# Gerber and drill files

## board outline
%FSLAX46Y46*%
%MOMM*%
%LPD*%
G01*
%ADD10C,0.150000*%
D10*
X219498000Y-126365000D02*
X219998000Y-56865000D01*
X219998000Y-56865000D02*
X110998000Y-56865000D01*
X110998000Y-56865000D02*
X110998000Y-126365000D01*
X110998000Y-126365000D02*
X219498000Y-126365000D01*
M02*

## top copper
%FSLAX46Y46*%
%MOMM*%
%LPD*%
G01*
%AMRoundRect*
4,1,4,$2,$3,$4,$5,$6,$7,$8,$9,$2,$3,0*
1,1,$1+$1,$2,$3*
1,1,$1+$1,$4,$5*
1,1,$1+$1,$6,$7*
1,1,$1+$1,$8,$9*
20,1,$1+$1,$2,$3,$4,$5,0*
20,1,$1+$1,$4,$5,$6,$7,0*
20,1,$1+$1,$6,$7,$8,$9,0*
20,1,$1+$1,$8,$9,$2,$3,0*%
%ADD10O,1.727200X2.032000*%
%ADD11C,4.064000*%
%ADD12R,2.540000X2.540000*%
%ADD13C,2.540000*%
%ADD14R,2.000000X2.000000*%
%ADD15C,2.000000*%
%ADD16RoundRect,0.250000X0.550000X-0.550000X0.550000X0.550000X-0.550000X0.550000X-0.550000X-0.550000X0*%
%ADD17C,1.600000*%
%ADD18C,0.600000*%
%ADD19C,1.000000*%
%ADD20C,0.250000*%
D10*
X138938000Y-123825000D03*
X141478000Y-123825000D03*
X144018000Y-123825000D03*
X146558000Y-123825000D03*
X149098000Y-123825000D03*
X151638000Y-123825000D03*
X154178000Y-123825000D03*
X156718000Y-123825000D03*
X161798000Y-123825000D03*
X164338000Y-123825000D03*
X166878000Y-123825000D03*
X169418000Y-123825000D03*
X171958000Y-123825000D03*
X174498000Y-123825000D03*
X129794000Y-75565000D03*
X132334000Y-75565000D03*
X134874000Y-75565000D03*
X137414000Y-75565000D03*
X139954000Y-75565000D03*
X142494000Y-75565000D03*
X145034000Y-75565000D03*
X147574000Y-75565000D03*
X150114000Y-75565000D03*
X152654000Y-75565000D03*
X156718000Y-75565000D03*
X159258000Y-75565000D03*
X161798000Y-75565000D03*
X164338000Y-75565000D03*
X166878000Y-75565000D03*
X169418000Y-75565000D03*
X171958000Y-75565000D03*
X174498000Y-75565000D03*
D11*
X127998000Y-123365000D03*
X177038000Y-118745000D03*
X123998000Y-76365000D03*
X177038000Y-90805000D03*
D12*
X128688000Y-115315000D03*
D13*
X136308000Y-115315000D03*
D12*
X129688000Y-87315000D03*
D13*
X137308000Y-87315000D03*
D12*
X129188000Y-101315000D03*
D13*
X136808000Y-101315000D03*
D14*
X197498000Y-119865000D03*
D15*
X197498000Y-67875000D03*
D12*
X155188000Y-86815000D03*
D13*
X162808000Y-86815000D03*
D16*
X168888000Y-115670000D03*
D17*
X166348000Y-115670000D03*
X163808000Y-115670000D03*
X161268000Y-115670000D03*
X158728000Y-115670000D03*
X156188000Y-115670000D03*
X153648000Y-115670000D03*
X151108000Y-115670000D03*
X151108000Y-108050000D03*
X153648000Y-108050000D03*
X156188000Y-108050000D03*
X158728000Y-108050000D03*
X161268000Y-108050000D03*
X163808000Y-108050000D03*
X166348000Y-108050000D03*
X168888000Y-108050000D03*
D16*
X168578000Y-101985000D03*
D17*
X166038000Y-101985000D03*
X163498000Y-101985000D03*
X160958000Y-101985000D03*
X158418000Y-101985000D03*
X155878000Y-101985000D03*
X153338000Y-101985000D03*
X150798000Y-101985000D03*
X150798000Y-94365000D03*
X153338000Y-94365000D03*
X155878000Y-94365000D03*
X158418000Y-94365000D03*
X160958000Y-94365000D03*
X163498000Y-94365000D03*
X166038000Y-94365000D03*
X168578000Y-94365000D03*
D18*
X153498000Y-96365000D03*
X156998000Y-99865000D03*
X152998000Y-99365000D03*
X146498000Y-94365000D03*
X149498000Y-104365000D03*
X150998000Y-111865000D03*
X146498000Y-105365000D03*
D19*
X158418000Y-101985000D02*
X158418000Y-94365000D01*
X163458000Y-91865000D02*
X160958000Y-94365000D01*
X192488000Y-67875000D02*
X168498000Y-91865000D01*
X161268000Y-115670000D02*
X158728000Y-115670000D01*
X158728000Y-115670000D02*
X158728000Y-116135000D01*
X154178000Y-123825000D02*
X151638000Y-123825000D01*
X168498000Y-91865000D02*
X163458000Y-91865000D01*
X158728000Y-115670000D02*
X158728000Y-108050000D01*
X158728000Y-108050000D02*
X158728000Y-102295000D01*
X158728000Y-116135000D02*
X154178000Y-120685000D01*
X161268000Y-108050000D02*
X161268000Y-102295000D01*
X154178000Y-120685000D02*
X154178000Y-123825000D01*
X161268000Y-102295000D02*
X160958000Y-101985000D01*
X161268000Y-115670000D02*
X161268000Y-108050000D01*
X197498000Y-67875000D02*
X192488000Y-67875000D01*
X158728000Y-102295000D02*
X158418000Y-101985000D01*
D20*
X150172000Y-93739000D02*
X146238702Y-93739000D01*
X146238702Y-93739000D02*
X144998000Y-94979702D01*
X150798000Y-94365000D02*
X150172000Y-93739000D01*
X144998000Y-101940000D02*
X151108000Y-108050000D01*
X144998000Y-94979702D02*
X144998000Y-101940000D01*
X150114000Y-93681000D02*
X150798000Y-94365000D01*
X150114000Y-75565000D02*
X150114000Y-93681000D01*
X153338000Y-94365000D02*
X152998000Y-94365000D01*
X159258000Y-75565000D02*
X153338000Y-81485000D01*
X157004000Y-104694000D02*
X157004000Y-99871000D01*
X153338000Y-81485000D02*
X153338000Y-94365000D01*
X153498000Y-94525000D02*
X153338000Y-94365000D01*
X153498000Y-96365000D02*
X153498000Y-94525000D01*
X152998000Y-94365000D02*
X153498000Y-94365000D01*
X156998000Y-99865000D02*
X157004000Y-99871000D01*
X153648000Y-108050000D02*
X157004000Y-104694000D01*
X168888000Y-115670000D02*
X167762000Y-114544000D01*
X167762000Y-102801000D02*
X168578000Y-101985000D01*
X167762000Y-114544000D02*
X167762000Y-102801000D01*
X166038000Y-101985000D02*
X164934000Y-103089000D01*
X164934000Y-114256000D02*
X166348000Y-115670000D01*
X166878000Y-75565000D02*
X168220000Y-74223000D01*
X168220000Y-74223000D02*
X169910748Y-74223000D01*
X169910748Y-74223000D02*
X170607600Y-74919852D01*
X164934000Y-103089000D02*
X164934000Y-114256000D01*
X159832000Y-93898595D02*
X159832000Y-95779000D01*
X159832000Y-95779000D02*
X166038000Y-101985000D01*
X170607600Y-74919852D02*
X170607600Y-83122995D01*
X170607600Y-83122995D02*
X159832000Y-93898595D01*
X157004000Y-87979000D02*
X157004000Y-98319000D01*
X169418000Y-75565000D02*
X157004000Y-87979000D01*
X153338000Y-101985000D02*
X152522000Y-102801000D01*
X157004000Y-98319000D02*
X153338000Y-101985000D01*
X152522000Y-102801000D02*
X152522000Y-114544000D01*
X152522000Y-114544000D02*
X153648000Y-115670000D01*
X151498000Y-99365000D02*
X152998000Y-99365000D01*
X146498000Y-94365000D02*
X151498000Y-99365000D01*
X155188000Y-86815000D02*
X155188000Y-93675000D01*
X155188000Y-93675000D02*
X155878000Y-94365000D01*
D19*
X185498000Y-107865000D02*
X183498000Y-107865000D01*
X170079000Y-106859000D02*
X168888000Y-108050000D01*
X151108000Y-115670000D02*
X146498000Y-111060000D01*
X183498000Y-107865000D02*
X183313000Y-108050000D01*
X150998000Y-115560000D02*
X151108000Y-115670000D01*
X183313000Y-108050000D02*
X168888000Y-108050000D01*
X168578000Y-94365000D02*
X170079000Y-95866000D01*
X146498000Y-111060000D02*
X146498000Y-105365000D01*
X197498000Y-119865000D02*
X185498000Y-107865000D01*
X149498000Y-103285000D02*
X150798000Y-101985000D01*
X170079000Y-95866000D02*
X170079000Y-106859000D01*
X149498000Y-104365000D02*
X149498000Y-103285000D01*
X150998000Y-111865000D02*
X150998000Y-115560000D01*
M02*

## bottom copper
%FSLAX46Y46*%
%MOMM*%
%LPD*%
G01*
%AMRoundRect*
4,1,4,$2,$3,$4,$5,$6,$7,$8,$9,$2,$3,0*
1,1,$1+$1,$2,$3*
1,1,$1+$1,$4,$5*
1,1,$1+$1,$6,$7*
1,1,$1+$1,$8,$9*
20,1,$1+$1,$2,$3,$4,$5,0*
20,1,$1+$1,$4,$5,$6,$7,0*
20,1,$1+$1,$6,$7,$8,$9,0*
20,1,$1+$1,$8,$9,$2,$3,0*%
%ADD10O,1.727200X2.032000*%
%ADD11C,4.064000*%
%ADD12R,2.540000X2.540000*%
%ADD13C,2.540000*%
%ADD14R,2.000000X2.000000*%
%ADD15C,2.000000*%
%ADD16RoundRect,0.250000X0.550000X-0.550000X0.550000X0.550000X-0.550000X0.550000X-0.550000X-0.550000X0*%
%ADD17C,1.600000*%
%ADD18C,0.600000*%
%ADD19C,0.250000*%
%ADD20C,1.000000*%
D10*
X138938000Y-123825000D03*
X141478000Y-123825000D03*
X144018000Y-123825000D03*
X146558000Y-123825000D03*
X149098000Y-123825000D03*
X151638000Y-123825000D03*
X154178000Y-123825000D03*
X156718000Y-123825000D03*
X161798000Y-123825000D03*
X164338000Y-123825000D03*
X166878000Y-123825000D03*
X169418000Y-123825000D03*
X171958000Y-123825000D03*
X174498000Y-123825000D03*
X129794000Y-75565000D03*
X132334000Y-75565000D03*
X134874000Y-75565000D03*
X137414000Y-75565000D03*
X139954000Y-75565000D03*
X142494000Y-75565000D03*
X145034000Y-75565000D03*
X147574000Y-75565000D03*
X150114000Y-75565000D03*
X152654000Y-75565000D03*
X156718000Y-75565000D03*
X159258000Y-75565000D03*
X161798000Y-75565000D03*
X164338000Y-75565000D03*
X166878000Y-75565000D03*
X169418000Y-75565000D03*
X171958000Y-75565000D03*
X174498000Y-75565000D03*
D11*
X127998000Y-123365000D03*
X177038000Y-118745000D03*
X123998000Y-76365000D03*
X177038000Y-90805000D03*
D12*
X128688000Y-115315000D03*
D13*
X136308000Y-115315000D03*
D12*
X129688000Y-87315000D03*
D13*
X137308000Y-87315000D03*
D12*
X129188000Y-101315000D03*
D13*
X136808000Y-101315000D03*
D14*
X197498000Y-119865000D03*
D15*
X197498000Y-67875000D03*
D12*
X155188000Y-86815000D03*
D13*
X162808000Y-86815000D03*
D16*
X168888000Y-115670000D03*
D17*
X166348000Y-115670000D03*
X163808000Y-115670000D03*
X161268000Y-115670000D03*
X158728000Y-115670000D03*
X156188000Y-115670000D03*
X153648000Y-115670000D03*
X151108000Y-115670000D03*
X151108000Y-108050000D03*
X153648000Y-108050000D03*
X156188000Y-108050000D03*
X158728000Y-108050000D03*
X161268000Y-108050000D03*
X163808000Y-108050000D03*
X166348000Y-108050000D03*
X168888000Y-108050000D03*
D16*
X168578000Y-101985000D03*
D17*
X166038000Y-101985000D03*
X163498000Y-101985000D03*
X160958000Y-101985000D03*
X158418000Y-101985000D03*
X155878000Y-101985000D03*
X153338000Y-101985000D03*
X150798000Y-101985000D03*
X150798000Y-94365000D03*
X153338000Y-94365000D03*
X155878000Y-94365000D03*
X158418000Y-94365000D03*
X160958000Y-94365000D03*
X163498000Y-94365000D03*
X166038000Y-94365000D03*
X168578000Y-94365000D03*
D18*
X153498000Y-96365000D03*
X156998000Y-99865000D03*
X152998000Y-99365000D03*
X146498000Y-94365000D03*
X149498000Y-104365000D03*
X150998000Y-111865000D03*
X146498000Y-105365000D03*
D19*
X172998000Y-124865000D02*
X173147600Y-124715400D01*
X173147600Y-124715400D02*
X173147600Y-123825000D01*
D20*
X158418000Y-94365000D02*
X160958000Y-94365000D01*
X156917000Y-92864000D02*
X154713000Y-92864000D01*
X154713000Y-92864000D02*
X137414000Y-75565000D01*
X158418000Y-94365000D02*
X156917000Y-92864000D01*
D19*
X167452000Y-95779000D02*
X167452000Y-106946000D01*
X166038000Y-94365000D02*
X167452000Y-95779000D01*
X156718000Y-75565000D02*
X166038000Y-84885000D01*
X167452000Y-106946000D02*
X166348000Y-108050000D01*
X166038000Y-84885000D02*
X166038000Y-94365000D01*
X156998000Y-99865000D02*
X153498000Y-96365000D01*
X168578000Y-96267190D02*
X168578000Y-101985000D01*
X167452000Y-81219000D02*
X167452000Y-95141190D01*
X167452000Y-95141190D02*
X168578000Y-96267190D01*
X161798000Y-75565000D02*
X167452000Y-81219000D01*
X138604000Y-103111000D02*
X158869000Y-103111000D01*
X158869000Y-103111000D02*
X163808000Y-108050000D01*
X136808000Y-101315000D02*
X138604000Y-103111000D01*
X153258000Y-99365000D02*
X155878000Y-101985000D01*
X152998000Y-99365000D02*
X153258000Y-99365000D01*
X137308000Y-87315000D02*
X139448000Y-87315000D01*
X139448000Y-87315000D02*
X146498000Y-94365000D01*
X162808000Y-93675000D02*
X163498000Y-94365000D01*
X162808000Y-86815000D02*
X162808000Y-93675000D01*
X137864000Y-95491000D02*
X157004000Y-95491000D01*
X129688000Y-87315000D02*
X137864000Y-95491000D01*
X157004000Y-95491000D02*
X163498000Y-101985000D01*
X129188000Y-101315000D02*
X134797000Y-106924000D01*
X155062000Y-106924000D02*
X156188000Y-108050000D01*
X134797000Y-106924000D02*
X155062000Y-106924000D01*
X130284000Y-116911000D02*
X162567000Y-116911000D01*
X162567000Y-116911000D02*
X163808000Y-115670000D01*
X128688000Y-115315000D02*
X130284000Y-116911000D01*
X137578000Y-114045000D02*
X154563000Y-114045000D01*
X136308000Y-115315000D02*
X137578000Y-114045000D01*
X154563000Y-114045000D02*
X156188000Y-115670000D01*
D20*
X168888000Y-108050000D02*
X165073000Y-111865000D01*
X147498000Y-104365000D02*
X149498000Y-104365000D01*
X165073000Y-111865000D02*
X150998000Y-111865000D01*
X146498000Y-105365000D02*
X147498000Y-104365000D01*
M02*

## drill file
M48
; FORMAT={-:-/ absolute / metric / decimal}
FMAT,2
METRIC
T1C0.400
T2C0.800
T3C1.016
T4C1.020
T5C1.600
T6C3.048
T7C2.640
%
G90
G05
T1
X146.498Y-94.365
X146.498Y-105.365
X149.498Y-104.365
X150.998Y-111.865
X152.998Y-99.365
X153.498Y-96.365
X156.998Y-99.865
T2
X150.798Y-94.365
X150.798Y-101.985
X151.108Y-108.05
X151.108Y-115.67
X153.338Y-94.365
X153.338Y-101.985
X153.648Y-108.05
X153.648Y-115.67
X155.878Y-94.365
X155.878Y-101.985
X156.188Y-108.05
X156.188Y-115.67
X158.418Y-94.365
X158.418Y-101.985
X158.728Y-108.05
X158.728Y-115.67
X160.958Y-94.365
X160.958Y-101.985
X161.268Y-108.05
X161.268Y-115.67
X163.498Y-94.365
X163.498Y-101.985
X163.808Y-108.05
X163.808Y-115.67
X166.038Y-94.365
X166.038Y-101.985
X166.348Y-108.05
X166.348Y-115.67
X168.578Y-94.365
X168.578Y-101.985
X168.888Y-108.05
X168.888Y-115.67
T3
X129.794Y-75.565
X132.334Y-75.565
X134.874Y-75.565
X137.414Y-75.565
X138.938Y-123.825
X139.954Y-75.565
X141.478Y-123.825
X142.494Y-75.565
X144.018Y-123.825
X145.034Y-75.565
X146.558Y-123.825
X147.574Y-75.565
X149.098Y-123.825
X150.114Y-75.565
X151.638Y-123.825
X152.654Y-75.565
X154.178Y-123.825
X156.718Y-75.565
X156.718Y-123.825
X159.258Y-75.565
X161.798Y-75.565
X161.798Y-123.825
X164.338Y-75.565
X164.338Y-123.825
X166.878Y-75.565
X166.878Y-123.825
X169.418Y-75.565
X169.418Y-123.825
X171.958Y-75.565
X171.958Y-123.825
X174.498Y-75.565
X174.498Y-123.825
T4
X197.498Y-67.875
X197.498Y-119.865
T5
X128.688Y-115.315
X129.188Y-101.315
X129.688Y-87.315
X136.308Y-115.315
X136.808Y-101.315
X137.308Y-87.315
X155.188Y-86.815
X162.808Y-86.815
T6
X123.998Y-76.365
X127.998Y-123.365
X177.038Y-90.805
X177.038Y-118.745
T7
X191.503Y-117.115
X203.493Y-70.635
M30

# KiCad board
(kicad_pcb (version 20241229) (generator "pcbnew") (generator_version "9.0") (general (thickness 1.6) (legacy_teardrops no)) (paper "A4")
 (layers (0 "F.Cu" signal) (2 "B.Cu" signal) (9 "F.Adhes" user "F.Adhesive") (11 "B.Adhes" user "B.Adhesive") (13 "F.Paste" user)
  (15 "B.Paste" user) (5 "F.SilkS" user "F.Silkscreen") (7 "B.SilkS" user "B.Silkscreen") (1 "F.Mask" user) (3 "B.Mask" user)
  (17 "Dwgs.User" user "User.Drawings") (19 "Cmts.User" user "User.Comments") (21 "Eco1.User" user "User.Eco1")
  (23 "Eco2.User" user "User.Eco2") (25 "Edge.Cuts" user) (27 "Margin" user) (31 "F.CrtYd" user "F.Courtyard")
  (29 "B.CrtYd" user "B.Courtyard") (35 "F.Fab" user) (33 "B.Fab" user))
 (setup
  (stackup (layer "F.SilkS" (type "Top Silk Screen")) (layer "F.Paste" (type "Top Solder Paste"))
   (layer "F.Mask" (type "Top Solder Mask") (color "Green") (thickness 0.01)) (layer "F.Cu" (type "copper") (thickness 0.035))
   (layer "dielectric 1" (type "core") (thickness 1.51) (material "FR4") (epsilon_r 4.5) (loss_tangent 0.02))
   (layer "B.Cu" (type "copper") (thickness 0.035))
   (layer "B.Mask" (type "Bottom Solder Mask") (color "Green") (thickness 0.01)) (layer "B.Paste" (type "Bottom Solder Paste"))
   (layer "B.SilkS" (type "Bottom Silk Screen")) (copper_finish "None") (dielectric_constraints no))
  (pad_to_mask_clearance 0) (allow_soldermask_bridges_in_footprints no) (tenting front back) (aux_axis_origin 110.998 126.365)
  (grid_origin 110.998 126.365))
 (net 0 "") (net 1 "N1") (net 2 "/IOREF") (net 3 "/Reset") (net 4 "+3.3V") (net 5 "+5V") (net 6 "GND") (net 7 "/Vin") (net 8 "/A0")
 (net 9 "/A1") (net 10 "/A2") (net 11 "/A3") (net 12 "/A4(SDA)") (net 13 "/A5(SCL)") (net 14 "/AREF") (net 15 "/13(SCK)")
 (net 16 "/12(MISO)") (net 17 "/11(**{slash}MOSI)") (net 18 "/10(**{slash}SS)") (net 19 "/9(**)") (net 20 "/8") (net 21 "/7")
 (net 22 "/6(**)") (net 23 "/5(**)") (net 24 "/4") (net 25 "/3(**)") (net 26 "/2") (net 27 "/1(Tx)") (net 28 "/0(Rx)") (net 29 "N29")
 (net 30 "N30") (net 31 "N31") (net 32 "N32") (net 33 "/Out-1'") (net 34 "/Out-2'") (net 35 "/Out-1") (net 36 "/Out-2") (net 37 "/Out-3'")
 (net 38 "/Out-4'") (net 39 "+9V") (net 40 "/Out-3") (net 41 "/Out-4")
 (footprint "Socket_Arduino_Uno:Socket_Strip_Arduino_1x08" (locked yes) (layer "F.Cu") (at 138.938 123.825)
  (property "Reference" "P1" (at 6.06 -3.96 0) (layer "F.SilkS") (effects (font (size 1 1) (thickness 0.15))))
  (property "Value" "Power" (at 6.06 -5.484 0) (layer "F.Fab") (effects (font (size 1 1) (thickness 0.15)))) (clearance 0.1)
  (pad "1" thru_hole oval (at 0 0) (size 1.7272 2.032) (drill 1.016) (layers "*.Cu" "*.Mask" "F.SilkS") (remove_unused_layers no)
   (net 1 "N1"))
  (pad "2" thru_hole oval (at 2.54 0) (size 1.7272 2.032) (drill 1.016) (layers "*.Cu" "*.Mask" "F.SilkS") (remove_unused_layers no)
   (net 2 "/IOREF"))
  (pad "3" thru_hole oval (at 5.08 0) (size 1.7272 2.032) (drill 1.016) (layers "*.Cu" "*.Mask" "F.SilkS") (remove_unused_layers no)
   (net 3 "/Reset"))
  (pad "4" thru_hole oval (at 7.62 0) (size 1.7272 2.032) (drill 1.016) (layers "*.Cu" "*.Mask" "F.SilkS") (remove_unused_layers no)
   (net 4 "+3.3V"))
  (pad "5" thru_hole oval (at 10.16 0) (size 1.7272 2.032) (drill 1.016) (layers "*.Cu" "*.Mask" "F.SilkS") (remove_unused_layers no)
   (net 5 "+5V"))
  (pad "6" thru_hole oval (at 12.7 0) (size 1.7272 2.032) (drill 1.016) (layers "*.Cu" "*.Mask" "F.SilkS") (remove_unused_layers no)
   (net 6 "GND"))
  (pad "7" thru_hole oval (at 15.24 0) (size 1.7272 2.032) (drill 1.016) (layers "*.Cu" "*.Mask" "F.SilkS") (remove_unused_layers no)
   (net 6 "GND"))
  (pad "8" thru_hole oval (at 17.78 0) (size 1.7272 2.032) (drill 1.016) (layers "*.Cu" "*.Mask" "F.SilkS") (remove_unused_layers no)
   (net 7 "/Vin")))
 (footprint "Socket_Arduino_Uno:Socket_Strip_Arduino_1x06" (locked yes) (layer "F.Cu") (at 161.798 123.825)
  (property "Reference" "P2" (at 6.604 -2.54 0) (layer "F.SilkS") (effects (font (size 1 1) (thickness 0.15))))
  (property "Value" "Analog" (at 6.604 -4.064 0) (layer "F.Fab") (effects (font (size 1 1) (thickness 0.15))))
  (pad "1" thru_hole oval (at 0 0) (size 1.7272 2.032) (drill 1.016) (layers "*.Cu" "*.Mask" "F.SilkS") (remove_unused_layers no)
   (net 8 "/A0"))
  (pad "2" thru_hole oval (at 2.54 0) (size 1.7272 2.032) (drill 1.016) (layers "*.Cu" "*.Mask" "F.SilkS") (remove_unused_layers no)
   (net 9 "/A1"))
  (pad "3" thru_hole oval (at 5.08 0) (size 1.7272 2.032) (drill 1.016) (layers "*.Cu" "*.Mask" "F.SilkS") (remove_unused_layers no)
   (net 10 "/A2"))
  (pad "4" thru_hole oval (at 7.62 0) (size 1.7272 2.032) (drill 1.016) (layers "*.Cu" "*.Mask" "F.SilkS") (remove_unused_layers no)
   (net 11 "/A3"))
  (pad "5" thru_hole oval (at 10.16 0) (size 1.7272 2.032) (drill 1.016) (layers "*.Cu" "*.Mask" "F.SilkS") (remove_unused_layers no)
   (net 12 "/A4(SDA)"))
  (pad "6" thru_hole oval (at 12.7 0) (size 1.7272 2.032) (drill 1.016) (layers "*.Cu" "*.Mask" "F.SilkS") (remove_unused_layers no)
   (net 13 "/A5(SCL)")))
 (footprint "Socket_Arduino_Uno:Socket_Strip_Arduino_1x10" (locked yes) (layer "F.Cu") (at 129.794 75.565)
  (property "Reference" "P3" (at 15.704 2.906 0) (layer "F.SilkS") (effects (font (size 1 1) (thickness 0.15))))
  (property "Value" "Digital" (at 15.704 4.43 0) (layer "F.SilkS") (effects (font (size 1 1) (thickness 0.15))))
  (pad "1" thru_hole oval (at 0 0) (size 1.7272 2.032) (drill 1.016) (layers "*.Cu" "*.Mask" "F.SilkS") (remove_unused_layers no))
  (pad "2" thru_hole oval (at 2.54 0) (size 1.7272 2.032) (drill 1.016) (layers "*.Cu" "*.Mask" "F.SilkS") (remove_unused_layers no))
  (pad "3" thru_hole oval (at 5.08 0) (size 1.7272 2.032) (drill 1.016) (layers "*.Cu" "*.Mask" "F.SilkS") (remove_unused_layers no)
   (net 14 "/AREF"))
  (pad "4" thru_hole oval (at 7.62 0) (size 1.7272 2.032) (drill 1.016) (layers "*.Cu" "*.Mask" "F.SilkS") (remove_unused_layers no)
   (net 6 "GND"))
  (pad "5" thru_hole oval (at 10.16 0) (size 1.7272 2.032) (drill 1.016) (layers "*.Cu" "*.Mask" "F.SilkS") (remove_unused_layers no)
   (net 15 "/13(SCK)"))
  (pad "6" thru_hole oval (at 12.7 0) (size 1.7272 2.032) (drill 1.016) (layers "*.Cu" "*.Mask" "F.SilkS") (remove_unused_layers no)
   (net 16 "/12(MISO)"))
  (pad "7" thru_hole oval (at 15.24 0) (size 1.7272 2.032) (drill 1.016) (layers "*.Cu" "*.Mask" "F.SilkS") (remove_unused_layers no)
   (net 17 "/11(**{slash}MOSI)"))
  (pad "8" thru_hole oval (at 17.78 0) (size 1.7272 2.032) (drill 1.016) (layers "*.Cu" "*.Mask" "F.SilkS") (remove_unused_layers no)
   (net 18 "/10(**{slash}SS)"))
  (pad "9" thru_hole oval (at 20.32 0) (size 1.7272 2.032) (drill 1.016) (layers "*.Cu" "*.Mask" "F.SilkS") (remove_unused_layers no)
   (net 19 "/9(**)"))
  (pad "10" thru_hole oval (at 22.86 0) (size 1.7272 2.032) (drill 1.016) (layers "*.Cu" "*.Mask" "F.SilkS") (remove_unused_layers no)
   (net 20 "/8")))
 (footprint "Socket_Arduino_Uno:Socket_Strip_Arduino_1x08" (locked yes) (layer "F.Cu") (at 156.718 75.565)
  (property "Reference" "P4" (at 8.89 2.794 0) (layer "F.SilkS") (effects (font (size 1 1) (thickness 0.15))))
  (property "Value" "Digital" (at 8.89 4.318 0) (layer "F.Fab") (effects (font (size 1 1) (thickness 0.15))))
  (pad "1" thru_hole oval (at 0 0) (size 1.7272 2.032) (drill 1.016) (layers "*.Cu" "*.Mask" "F.SilkS") (remove_unused_layers no)
   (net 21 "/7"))
  (pad "2" thru_hole oval (at 2.54 0) (size 1.7272 2.032) (drill 1.016) (layers "*.Cu" "*.Mask" "F.SilkS") (remove_unused_layers no)
   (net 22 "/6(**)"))
  (pad "3" thru_hole oval (at 5.08 0) (size 1.7272 2.032) (drill 1.016) (layers "*.Cu" "*.Mask" "F.SilkS") (remove_unused_layers no)
   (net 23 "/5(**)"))
  (pad "4" thru_hole oval (at 7.62 0) (size 1.7272 2.032) (drill 1.016) (layers "*.Cu" "*.Mask" "F.SilkS") (remove_unused_layers no)
   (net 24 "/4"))
  (pad "5" thru_hole oval (at 10.16 0) (size 1.7272 2.032) (drill 1.016) (layers "*.Cu" "*.Mask" "F.SilkS") (remove_unused_layers no)
   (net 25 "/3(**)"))
  (pad "6" thru_hole oval (at 12.7 0) (size 1.7272 2.032) (drill 1.016) (layers "*.Cu" "*.Mask" "F.SilkS") (remove_unused_layers no)
   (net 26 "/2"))
  (pad "7" thru_hole oval (at 15.24 0) (size 1.7272 2.032) (drill 1.016) (layers "*.Cu" "*.Mask" "F.SilkS") (remove_unused_layers no)
   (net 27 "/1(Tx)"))
  (pad "8" thru_hole oval (at 17.78 0) (size 1.7272 2.032) (drill 1.016) (layers "*.Cu" "*.Mask" "F.SilkS") (remove_unused_layers no)
   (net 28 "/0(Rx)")))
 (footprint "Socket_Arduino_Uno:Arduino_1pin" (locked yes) (layer "F.Cu") (at 127.998 123.365)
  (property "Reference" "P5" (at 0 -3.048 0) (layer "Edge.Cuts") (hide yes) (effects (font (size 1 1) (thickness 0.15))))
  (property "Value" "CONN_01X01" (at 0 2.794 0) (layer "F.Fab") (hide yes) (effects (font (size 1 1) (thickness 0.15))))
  (pad "1" thru_hole circle (at 0 0) (size 4.064 4.064) (drill 3.048) (layers "*.Cu" "*.Mask" "F.SilkS") (remove_unused_layers no)
   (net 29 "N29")))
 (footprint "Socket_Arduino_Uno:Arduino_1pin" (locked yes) (layer "F.Cu") (at 177.038 118.745)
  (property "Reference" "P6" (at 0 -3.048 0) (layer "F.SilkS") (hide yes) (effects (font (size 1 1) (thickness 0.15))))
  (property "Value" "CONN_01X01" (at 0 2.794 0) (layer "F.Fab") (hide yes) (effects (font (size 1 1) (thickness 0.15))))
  (pad "1" thru_hole circle (at 0 0) (size 4.064 4.064) (drill 3.048) (layers "*.Cu" "*.Mask" "F.SilkS") (remove_unused_layers no)
   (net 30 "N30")))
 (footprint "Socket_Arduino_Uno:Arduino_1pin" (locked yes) (layer "F.Cu") (at 123.998 76.365)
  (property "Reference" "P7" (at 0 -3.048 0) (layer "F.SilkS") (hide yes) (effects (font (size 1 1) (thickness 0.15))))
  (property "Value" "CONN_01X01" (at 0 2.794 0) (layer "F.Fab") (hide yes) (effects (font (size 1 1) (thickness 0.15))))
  (pad "1" thru_hole circle (at 0 0) (size 4.064 4.064) (drill 3.048) (layers "*.Cu" "*.Mask" "F.SilkS") (remove_unused_layers no)
   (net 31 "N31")))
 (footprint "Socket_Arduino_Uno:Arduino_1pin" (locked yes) (layer "F.Cu") (at 177.038 90.805)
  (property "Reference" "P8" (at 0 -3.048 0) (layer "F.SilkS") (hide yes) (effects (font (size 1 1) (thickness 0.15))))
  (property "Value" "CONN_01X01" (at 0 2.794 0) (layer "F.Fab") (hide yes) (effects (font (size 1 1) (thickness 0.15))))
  (pad "1" thru_hole circle (at 0 0) (size 4.064 4.064) (drill 3.048) (layers "*.Cu" "*.Mask" "F.SilkS") (remove_unused_layers no)
   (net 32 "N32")))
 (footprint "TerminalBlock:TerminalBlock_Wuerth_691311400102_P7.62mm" (layer "F.Cu") (at 128.688 115.315)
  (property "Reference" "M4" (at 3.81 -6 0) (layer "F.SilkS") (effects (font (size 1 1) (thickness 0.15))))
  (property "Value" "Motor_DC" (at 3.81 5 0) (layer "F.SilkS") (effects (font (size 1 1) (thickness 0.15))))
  (pad "1" thru_hole rect (at 0 0) (size 2.54 2.54) (drill 1.6) (layers "*.Cu" "*.Mask") (remove_unused_layers no) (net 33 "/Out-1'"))
  (pad "2" thru_hole circle (at 7.62 0) (size 2.54 2.54) (drill 1.6) (layers "*.Cu" "*.Mask") (remove_unused_layers no) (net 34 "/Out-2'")))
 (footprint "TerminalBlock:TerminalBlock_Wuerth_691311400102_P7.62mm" (layer "F.Cu") (at 129.688 87.315)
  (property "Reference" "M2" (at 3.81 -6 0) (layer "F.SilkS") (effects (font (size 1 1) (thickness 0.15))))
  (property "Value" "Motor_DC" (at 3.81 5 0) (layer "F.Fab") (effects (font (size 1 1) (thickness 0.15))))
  (pad "1" thru_hole rect (at 0 0) (size 2.54 2.54) (drill 1.6) (layers "*.Cu" "*.Mask") (remove_unused_layers no) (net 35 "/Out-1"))
  (pad "2" thru_hole circle (at 7.62 0) (size 2.54 2.54) (drill 1.6) (layers "*.Cu" "*.Mask") (remove_unused_layers no) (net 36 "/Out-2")))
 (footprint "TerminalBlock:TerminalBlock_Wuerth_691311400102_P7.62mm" (layer "F.Cu") (at 129.188 101.315)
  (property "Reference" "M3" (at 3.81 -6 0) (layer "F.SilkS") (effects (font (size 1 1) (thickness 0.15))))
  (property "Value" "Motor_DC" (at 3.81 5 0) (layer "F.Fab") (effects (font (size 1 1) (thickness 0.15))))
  (pad "1" thru_hole rect (at 0 0) (size 2.54 2.54) (drill 1.6) (layers "*.Cu" "*.Mask") (remove_unused_layers no) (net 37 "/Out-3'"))
  (pad "2" thru_hole circle (at 7.62 0) (size 2.54 2.54) (drill 1.6) (layers "*.Cu" "*.Mask") (remove_unused_layers no) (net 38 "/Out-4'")))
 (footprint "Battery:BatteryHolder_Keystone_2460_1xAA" (layer "F.Cu") (at 197.498 119.865 90)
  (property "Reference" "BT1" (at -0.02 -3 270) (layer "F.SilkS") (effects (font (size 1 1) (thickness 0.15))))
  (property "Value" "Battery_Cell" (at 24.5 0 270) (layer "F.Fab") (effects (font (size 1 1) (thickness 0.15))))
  (pad "" np_thru_hole circle (at 2.75 -5.995 180) (size 2.64 2.64) (drill 2.64) (layers "*.Cu" "*.Mask"))
  (pad "" np_thru_hole circle (at 49.23 5.995 90) (size 2.64 2.64) (drill 2.64) (layers "*.Cu" "*.Mask"))
  (pad "1" thru_hole rect (at 0 0 270) (size 2 2) (drill 1.02) (layers "*.Cu" "*.Mask") (remove_unused_layers no) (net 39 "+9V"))
  (pad "2" thru_hole circle (at 51.99 0 270) (size 2 2) (drill 1.02) (layers "*.Cu" "*.Mask") (remove_unused_layers no) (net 6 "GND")))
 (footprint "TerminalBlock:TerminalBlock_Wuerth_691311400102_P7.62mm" (layer "F.Cu") (at 155.188 86.815)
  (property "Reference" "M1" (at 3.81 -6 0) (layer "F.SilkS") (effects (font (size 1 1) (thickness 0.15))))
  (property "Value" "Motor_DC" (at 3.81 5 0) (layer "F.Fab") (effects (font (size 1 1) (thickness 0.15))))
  (pad "1" thru_hole rect (at 0 0) (size 2.54 2.54) (drill 1.6) (layers "*.Cu" "*.Mask") (remove_unused_layers no) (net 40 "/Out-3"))
  (pad "2" thru_hole circle (at 7.62 0) (size 2.54 2.54) (drill 1.6) (layers "*.Cu" "*.Mask") (remove_unused_layers no) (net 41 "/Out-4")))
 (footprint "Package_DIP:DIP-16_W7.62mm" (layer "B.Cu") (at 168.888 115.67 90)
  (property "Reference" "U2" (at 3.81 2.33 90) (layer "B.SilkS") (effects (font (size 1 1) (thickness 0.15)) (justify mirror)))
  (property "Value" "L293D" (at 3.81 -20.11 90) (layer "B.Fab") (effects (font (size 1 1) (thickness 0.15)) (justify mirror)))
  (pad "1" thru_hole roundrect (at 0 0 90) (size 1.6 1.6) (drill 0.8) (layers "*.Cu" "*.Mask") (remove_unused_layers no)
   (roundrect_rratio 0.15625) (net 23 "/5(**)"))
  (pad "2" thru_hole circle (at 0 -2.54 90) (size 1.6 1.6) (drill 0.8) (layers "*.Cu" "*.Mask") (remove_unused_layers no) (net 25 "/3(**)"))
  (pad "3" thru_hole circle (at 0 -5.08 90) (size 1.6 1.6) (drill 0.8) (layers "*.Cu" "*.Mask") (remove_unused_layers no) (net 33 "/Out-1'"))
  (pad "4" thru_hole circle (at 0 -7.62 90) (size 1.6 1.6) (drill 0.8) (layers "*.Cu" "*.Mask") (remove_unused_layers no) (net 6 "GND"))
  (pad "5" thru_hole circle (at 0 -10.16 90) (size 1.6 1.6) (drill 0.8) (layers "*.Cu" "*.Mask") (remove_unused_layers no) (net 6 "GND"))
  (pad "6" thru_hole circle (at 0 -12.7 90) (size 1.6 1.6) (drill 0.8) (layers "*.Cu" "*.Mask") (remove_unused_layers no) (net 34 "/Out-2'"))
  (pad "7" thru_hole circle (at 0 -15.24 90) (size 1.6 1.6) (drill 0.8) (layers "*.Cu" "*.Mask") (remove_unused_layers no) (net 26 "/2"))
  (pad "8" thru_hole circle (at 0 -17.78 90) (size 1.6 1.6) (drill 0.8) (layers "*.Cu" "*.Mask") (remove_unused_layers no) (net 39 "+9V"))
  (pad "9" thru_hole circle (at 7.62 -17.78 90) (size 1.6 1.6) (drill 0.8) (layers "*.Cu" "*.Mask") (remove_unused_layers no)
   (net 19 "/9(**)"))
  (pad "10" thru_hole circle (at 7.62 -15.24 90) (size 1.6 1.6) (drill 0.8) (layers "*.Cu" "*.Mask") (remove_unused_layers no)
   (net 22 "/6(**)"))
  (pad "11" thru_hole circle (at 7.62 -12.7 90) (size 1.6 1.6) (drill 0.8) (layers "*.Cu" "*.Mask") (remove_unused_layers no)
   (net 37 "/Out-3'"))
  (pad "12" thru_hole circle (at 7.62 -10.16 90) (size 1.6 1.6) (drill 0.8) (layers "*.Cu" "*.Mask") (remove_unused_layers no) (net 6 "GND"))
  (pad "13" thru_hole circle (at 7.62 -7.62 90) (size 1.6 1.6) (drill 0.8) (layers "*.Cu" "*.Mask") (remove_unused_layers no) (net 6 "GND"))
  (pad "14" thru_hole circle (at 7.62 -5.08 90) (size 1.6 1.6) (drill 0.8) (layers "*.Cu" "*.Mask") (remove_unused_layers no)
   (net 38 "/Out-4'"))
  (pad "15" thru_hole circle (at 7.62 -2.54 90) (size 1.6 1.6) (drill 0.8) (layers "*.Cu" "*.Mask") (remove_unused_layers no) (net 21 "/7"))
  (pad "16" thru_hole circle (at 7.62 0 90) (size 1.6 1.6) (drill 0.8) (layers "*.Cu" "*.Mask") (remove_unused_layers no) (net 39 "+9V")))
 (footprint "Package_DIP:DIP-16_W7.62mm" (layer "B.Cu") (at 168.578 101.985 90)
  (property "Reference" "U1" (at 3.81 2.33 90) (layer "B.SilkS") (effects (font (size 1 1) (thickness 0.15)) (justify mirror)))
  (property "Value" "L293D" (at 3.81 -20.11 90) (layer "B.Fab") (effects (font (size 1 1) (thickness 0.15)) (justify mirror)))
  (pad "1" thru_hole roundrect (at 0 0 90) (size 1.6 1.6) (drill 0.8) (layers "*.Cu" "*.Mask") (remove_unused_layers no)
   (roundrect_rratio 0.15625) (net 23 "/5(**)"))
  (pad "2" thru_hole circle (at 0 -2.54 90) (size 1.6 1.6) (drill 0.8) (layers "*.Cu" "*.Mask") (remove_unused_layers no) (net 25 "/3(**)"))
  (pad "3" thru_hole circle (at 0 -5.08 90) (size 1.6 1.6) (drill 0.8) (layers "*.Cu" "*.Mask") (remove_unused_layers no) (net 35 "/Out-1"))
  (pad "4" thru_hole circle (at 0 -7.62 90) (size 1.6 1.6) (drill 0.8) (layers "*.Cu" "*.Mask") (remove_unused_layers no) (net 6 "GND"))
  (pad "5" thru_hole circle (at 0 -10.16 90) (size 1.6 1.6) (drill 0.8) (layers "*.Cu" "*.Mask") (remove_unused_layers no) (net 6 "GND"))
  (pad "6" thru_hole circle (at 0 -12.7 90) (size 1.6 1.6) (drill 0.8) (layers "*.Cu" "*.Mask") (remove_unused_layers no) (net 36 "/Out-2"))
  (pad "7" thru_hole circle (at 0 -15.24 90) (size 1.6 1.6) (drill 0.8) (layers "*.Cu" "*.Mask") (remove_unused_layers no) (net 26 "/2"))
  (pad "8" thru_hole circle (at 0 -17.78 90) (size 1.6 1.6) (drill 0.8) (layers "*.Cu" "*.Mask") (remove_unused_layers no) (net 39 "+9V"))
  (pad "9" thru_hole circle (at 7.62 -17.78 90) (size 1.6 1.6) (drill 0.8) (layers "*.Cu" "*.Mask") (remove_unused_layers no)
   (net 19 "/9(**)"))
  (pad "10" thru_hole circle (at 7.62 -15.24 90) (size 1.6 1.6) (drill 0.8) (layers "*.Cu" "*.Mask") (remove_unused_layers no)
   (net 22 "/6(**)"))
  (pad "11" thru_hole circle (at 7.62 -12.7 90) (size 1.6 1.6) (drill 0.8) (layers "*.Cu" "*.Mask") (remove_unused_layers no)
   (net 40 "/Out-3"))
  (pad "12" thru_hole circle (at 7.62 -10.16 90) (size 1.6 1.6) (drill 0.8) (layers "*.Cu" "*.Mask") (remove_unused_layers no) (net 6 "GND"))
  (pad "13" thru_hole circle (at 7.62 -7.62 90) (size 1.6 1.6) (drill 0.8) (layers "*.Cu" "*.Mask") (remove_unused_layers no) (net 6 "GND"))
  (pad "14" thru_hole circle (at 7.62 -5.08 90) (size 1.6 1.6) (drill 0.8) (layers "*.Cu" "*.Mask") (remove_unused_layers no)
   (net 41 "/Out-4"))
  (pad "15" thru_hole circle (at 7.62 -2.54 90) (size 1.6 1.6) (drill 0.8) (layers "*.Cu" "*.Mask") (remove_unused_layers no) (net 21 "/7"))
  (pad "16" thru_hole circle (at 7.62 0 90) (size 1.6 1.6) (drill 0.8) (layers "*.Cu" "*.Mask") (remove_unused_layers no) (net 39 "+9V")))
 (gr_line (start 219.498 126.365) (end 219.998 56.865) (stroke (width 0.15) (type solid)) (layer "Edge.Cuts"))
 (gr_line (start 219.998 56.865) (end 110.998 56.865) (stroke (width 0.15) (type solid)) (layer "Edge.Cuts"))
 (gr_line (start 110.998 56.865) (end 110.998 126.365) (stroke (width 0.15) (type solid)) (layer "Edge.Cuts"))
 (gr_line (start 110.998 126.365) (end 219.498 126.365) (stroke (width 0.15) (type solid)) (layer "Edge.Cuts"))
 (segment (start 172.998 124.865) (end 173.1476 124.7154) (width 0.25) (layer "B.Cu") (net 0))
 (segment (start 173.1476 124.7154) (end 173.1476 123.825) (width 0.25) (layer "B.Cu") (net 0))
 (segment (start 158.418 101.985) (end 158.418 94.365) (width 1) (layer "F.Cu") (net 6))
 (segment (start 163.458 91.865) (end 160.958 94.365) (width 1) (layer "F.Cu") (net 6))
 (segment (start 192.488 67.875) (end 168.498 91.865) (width 1) (layer "F.Cu") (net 6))
 (segment (start 161.268 115.67) (end 158.728 115.67) (width 1) (layer "F.Cu") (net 6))
 (segment (start 158.728 115.67) (end 158.728 116.135) (width 1) (layer "F.Cu") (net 6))
 (segment (start 154.178 123.825) (end 151.638 123.825) (width 1) (layer "F.Cu") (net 6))
 (segment (start 168.498 91.865) (end 163.458 91.865) (width 1) (layer "F.Cu") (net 6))
 (segment (start 158.728 115.67) (end 158.728 108.05) (width 1) (layer "F.Cu") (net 6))
 (segment (start 158.728 108.05) (end 158.728 102.295) (width 1) (layer "F.Cu") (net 6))
 (segment (start 158.728 116.135) (end 154.178 120.685) (width 1) (layer "F.Cu") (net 6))
 (segment (start 161.268 108.05) (end 161.268 102.295) (width 1) (layer "F.Cu") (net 6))
 (segment (start 154.178 120.685) (end 154.178 123.825) (width 1) (layer "F.Cu") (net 6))
 (segment (start 161.268 102.295) (end 160.958 101.985) (width 1) (layer "F.Cu") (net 6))
 (segment (start 161.268 115.67) (end 161.268 108.05) (width 1) (layer "F.Cu") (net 6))
 (segment (start 197.498 67.875) (end 192.488 67.875) (width 1) (layer "F.Cu") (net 6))
 (segment (start 158.728 102.295) (end 158.418 101.985) (width 1) (layer "F.Cu") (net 6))
 (segment (start 158.418 94.365) (end 160.958 94.365) (width 1) (layer "B.Cu") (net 6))
 (segment (start 156.917 92.864) (end 154.713 92.864) (width 1) (layer "B.Cu") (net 6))
 (segment (start 154.713 92.864) (end 137.414 75.565) (width 1) (layer "B.Cu") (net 6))
 (segment (start 158.418 94.365) (end 156.917 92.864) (width 1) (layer "B.Cu") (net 6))
 (segment (start 150.172 93.739) (end 146.238702 93.739) (width 0.25) (layer "F.Cu") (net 19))
 (segment (start 146.238702 93.739) (end 144.998 94.979702) (width 0.25) (layer "F.Cu") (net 19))
 (segment (start 150.798 94.365) (end 150.172 93.739) (width 0.25) (layer "F.Cu") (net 19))
 (segment (start 144.998 101.94) (end 151.108 108.05) (width 0.25) (layer "F.Cu") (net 19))
 (segment (start 144.998 94.979702) (end 144.998 101.94) (width 0.25) (layer "F.Cu") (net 19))
 (segment (start 150.114 93.681) (end 150.798 94.365) (width 0.25) (layer "F.Cu") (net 19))
 (segment (start 150.114 75.565) (end 150.114 93.681) (width 0.25) (layer "F.Cu") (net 19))
 (segment (start 167.452 95.779) (end 167.452 106.946) (width 0.25) (layer "B.Cu") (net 21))
 (segment (start 166.038 94.365) (end 167.452 95.779) (width 0.25) (layer "B.Cu") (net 21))
 (segment (start 156.718 75.565) (end 166.038 84.885) (width 0.25) (layer "B.Cu") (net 21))
 (segment (start 167.452 106.946) (end 166.348 108.05) (width 0.25) (layer "B.Cu") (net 21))
 (segment (start 166.038 84.885) (end 166.038 94.365) (width 0.25) (layer "B.Cu") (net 21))
 (segment (start 153.338 94.365) (end 152.998 94.365) (width 0.25) (layer "F.Cu") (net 22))
 (segment (start 159.258 75.565) (end 153.338 81.485) (width 0.25) (layer "F.Cu") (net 22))
 (segment (start 157.004 104.694) (end 157.004 99.871) (width 0.25) (layer "F.Cu") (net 22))
 (segment (start 153.338 81.485) (end 153.338 94.365) (width 0.25) (layer "F.Cu") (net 22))
 (segment (start 153.498 94.525) (end 153.338 94.365) (width 0.25) (layer "F.Cu") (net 22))
 (segment (start 153.498 96.365) (end 153.498 94.525) (width 0.25) (layer "F.Cu") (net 22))
 (segment (start 152.998 94.365) (end 153.498 94.365) (width 0.25) (layer "F.Cu") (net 22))
 (segment (start 156.998 99.865) (end 157.004 99.871) (width 0.25) (layer "F.Cu") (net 22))
 (segment (start 153.648 108.05) (end 157.004 104.694) (width 0.25) (layer "F.Cu") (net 22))
 (via (at 153.498 96.365) (size 0.6) (drill 0.4) (layers "F.Cu" "B.Cu") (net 22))
 (via (at 156.998 99.865) (size 0.6) (drill 0.4) (layers "F.Cu" "B.Cu") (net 22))
 (segment (start 156.998 99.865) (end 153.498 96.365) (width 0.25) (layer "B.Cu") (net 22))
 (segment (start 168.888 115.67) (end 167.762 114.544) (width 0.25) (layer "F.Cu") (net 23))
 (segment (start 167.762 102.801) (end 168.578 101.985) (width 0.25) (layer "F.Cu") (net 23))
 (segment (start 167.762 114.544) (end 167.762 102.801) (width 0.25) (layer "F.Cu") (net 23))
 (segment (start 168.578 96.26719) (end 168.578 101.985) (width 0.25) (layer "B.Cu") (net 23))
 (segment (start 167.452 81.219) (end 167.452 95.14119) (width 0.25) (layer "B.Cu") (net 23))
 (segment (start 167.452 95.14119) (end 168.578 96.26719) (width 0.25) (layer "B.Cu") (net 23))
 (segment (start 161.798 75.565) (end 167.452 81.219) (width 0.25) (layer "B.Cu") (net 23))
 (segment (start 166.038 101.985) (end 164.934 103.089) (width 0.25) (layer "F.Cu") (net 25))
 (segment (start 164.934 114.256) (end 166.348 115.67) (width 0.25) (layer "F.Cu") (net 25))
 (segment (start 166.878 75.565) (end 168.22 74.223) (width 0.25) (layer "F.Cu") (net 25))
 (segment (start 168.22 74.223) (end 169.910748 74.223) (width 0.25) (layer "F.Cu") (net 25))
 (segment (start 169.910748 74.223) (end 170.6076 74.919852) (width 0.25) (layer "F.Cu") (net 25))
 (segment (start 164.934 103.089) (end 164.934 114.256) (width 0.25) (layer "F.Cu") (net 25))
 (segment (start 159.832 93.898595) (end 159.832 95.779) (width 0.25) (layer "F.Cu") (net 25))
 (segment (start 159.832 95.779) (end 166.038 101.985) (width 0.25) (layer "F.Cu") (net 25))
 (segment (start 170.6076 74.919852) (end 170.6076 83.122995) (width 0.25) (layer "F.Cu") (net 25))
 (segment (start 170.6076 83.122995) (end 159.832 93.898595) (width 0.25) (layer "F.Cu") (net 25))
 (segment (start 157.004 87.979) (end 157.004 98.319) (width 0.25) (layer "F.Cu") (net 26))
 (segment (start 169.418 75.565) (end 157.004 87.979) (width 0.25) (layer "F.Cu") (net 26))
 (segment (start 153.338 101.985) (end 152.522 102.801) (width 0.25) (layer "F.Cu") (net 26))
 (segment (start 157.004 98.319) (end 153.338 101.985) (width 0.25) (layer "F.Cu") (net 26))
 (segment (start 152.522 102.801) (end 152.522 114.544) (width 0.25) (layer "F.Cu") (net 26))
 (segment (start 152.522 114.544) (end 153.648 115.67) (width 0.25) (layer "F.Cu") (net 26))
 (segment (start 138.604 103.111) (end 158.869 103.111) (width 0.25) (layer "B.Cu") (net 38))
 (segment (start 158.869 103.111) (end 163.808 108.05) (width 0.25) (layer "B.Cu") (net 38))
 (segment (start 136.808 101.315) (end 138.604 103.111) (width 0.25) (layer "B.Cu") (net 38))
 (segment (start 151.498 99.365) (end 152.998 99.365) (width 0.25) (layer "F.Cu") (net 36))
 (segment (start 146.498 94.365) (end 151.498 99.365) (width 0.25) (layer "F.Cu") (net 36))
 (via (at 152.998 99.365) (size 0.6) (drill 0.4) (layers "F.Cu" "B.Cu") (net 36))
 (via (at 146.498 94.365) (size 0.6) (drill 0.4) (layers "F.Cu" "B.Cu") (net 36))
 (segment (start 153.258 99.365) (end 155.878 101.985) (width 0.25) (layer "B.Cu") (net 36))
 (segment (start 152.998 99.365) (end 153.258 99.365) (width 0.25) (layer "B.Cu") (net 36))
 (segment (start 137.308 87.315) (end 139.448 87.315) (width 0.25) (layer "B.Cu") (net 36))
 (segment (start 139.448 87.315) (end 146.498 94.365) (width 0.25) (layer "B.Cu") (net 36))
 (segment (start 162.808 93.675) (end 163.498 94.365) (width 0.25) (layer "B.Cu") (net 41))
 (segment (start 162.808 86.815) (end 162.808 93.675) (width 0.25) (layer "B.Cu") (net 41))
 (segment (start 137.864 95.491) (end 157.004 95.491) (width 0.25) (layer "B.Cu") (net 35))
 (segment (start 129.688 87.315) (end 137.864 95.491) (width 0.25) (layer "B.Cu") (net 35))
 (segment (start 157.004 95.491) (end 163.498 101.985) (width 0.25) (layer "B.Cu") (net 35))
 (segment (start 155.188 86.815) (end 155.188 93.675) (width 0.25) (layer "F.Cu") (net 40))
 (segment (start 155.188 93.675) (end 155.878 94.365) (width 0.25) (layer "F.Cu") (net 40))
 (segment (start 129.188 101.315) (end 134.797 106.924) (width 0.25) (layer "B.Cu") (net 37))
 (segment (start 155.062 106.924) (end 156.188 108.05) (width 0.25) (layer "B.Cu") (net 37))
 (segment (start 134.797 106.924) (end 155.062 106.924) (width 0.25) (layer "B.Cu") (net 37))
 (segment (start 130.284 116.911) (end 162.567 116.911) (width 0.25) (layer "B.Cu") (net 33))
 (segment (start 162.567 116.911) (end 163.808 115.67) (width 0.25) (layer "B.Cu") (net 33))
 (segment (start 128.688 115.315) (end 130.284 116.911) (width 0.25) (layer "B.Cu") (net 33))
 (segment (start 137.578 114.045) (end 154.563 114.045) (width 0.25) (layer "B.Cu") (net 34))
 (segment (start 136.308 115.315) (end 137.578 114.045) (width 0.25) (layer "B.Cu") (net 34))
 (segment (start 154.563 114.045) (end 156.188 115.67) (width 0.25) (layer "B.Cu") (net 34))
 (segment (start 185.498 107.865) (end 183.498 107.865) (width 1) (layer "F.Cu") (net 39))
 (segment (start 170.079 106.859) (end 168.888 108.05) (width 1) (layer "F.Cu") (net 39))
 (segment (start 151.108 115.67) (end 146.498 111.06) (width 1) (layer "F.Cu") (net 39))
 (segment (start 183.498 107.865) (end 183.313 108.05) (width 1) (layer "F.Cu") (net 39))
 (segment (start 150.998 115.56) (end 151.108 115.67) (width 1) (layer "F.Cu") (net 39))
 (segment (start 183.313 108.05) (end 168.888 108.05) (width 1) (layer "F.Cu") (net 39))
 (segment (start 168.578 94.365) (end 170.079 95.866) (width 1) (layer "F.Cu") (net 39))
 (segment (start 146.498 111.06) (end 146.498 105.365) (width 1) (layer "F.Cu") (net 39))
 (segment (start 197.498 119.865) (end 185.498 107.865) (width 1) (layer "F.Cu") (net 39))
 (segment (start 149.498 103.285) (end 150.798 101.985) (width 1) (layer "F.Cu") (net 39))
 (segment (start 170.079 95.866) (end 170.079 106.859) (width 1) (layer "F.Cu") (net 39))
 (segment (start 149.498 104.365) (end 149.498 103.285) (width 1) (layer "F.Cu") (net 39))
 (segment (start 150.998 111.865) (end 150.998 115.56) (width 1) (layer "F.Cu") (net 39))
 (via (at 149.498 104.365) (size 0.6) (drill 0.4) (layers "F.Cu" "B.Cu") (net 39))
 (via (at 150.998 111.865) (size 0.6) (drill 0.4) (layers "F.Cu" "B.Cu") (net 39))
 (via (at 146.498 105.365) (size 0.6) (drill 0.4) (layers "F.Cu" "B.Cu") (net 39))
 (segment (start 168.888 108.05) (end 165.073 111.865) (width 1) (layer "B.Cu") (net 39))
 (segment (start 147.498 104.365) (end 149.498 104.365) (width 1) (layer "B.Cu") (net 39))
 (segment (start 165.073 111.865) (end 150.998 111.865) (width 1) (layer "B.Cu") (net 39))
 (segment (start 146.498 105.365) (end 147.498 104.365) (width 1) (layer "B.Cu") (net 39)))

